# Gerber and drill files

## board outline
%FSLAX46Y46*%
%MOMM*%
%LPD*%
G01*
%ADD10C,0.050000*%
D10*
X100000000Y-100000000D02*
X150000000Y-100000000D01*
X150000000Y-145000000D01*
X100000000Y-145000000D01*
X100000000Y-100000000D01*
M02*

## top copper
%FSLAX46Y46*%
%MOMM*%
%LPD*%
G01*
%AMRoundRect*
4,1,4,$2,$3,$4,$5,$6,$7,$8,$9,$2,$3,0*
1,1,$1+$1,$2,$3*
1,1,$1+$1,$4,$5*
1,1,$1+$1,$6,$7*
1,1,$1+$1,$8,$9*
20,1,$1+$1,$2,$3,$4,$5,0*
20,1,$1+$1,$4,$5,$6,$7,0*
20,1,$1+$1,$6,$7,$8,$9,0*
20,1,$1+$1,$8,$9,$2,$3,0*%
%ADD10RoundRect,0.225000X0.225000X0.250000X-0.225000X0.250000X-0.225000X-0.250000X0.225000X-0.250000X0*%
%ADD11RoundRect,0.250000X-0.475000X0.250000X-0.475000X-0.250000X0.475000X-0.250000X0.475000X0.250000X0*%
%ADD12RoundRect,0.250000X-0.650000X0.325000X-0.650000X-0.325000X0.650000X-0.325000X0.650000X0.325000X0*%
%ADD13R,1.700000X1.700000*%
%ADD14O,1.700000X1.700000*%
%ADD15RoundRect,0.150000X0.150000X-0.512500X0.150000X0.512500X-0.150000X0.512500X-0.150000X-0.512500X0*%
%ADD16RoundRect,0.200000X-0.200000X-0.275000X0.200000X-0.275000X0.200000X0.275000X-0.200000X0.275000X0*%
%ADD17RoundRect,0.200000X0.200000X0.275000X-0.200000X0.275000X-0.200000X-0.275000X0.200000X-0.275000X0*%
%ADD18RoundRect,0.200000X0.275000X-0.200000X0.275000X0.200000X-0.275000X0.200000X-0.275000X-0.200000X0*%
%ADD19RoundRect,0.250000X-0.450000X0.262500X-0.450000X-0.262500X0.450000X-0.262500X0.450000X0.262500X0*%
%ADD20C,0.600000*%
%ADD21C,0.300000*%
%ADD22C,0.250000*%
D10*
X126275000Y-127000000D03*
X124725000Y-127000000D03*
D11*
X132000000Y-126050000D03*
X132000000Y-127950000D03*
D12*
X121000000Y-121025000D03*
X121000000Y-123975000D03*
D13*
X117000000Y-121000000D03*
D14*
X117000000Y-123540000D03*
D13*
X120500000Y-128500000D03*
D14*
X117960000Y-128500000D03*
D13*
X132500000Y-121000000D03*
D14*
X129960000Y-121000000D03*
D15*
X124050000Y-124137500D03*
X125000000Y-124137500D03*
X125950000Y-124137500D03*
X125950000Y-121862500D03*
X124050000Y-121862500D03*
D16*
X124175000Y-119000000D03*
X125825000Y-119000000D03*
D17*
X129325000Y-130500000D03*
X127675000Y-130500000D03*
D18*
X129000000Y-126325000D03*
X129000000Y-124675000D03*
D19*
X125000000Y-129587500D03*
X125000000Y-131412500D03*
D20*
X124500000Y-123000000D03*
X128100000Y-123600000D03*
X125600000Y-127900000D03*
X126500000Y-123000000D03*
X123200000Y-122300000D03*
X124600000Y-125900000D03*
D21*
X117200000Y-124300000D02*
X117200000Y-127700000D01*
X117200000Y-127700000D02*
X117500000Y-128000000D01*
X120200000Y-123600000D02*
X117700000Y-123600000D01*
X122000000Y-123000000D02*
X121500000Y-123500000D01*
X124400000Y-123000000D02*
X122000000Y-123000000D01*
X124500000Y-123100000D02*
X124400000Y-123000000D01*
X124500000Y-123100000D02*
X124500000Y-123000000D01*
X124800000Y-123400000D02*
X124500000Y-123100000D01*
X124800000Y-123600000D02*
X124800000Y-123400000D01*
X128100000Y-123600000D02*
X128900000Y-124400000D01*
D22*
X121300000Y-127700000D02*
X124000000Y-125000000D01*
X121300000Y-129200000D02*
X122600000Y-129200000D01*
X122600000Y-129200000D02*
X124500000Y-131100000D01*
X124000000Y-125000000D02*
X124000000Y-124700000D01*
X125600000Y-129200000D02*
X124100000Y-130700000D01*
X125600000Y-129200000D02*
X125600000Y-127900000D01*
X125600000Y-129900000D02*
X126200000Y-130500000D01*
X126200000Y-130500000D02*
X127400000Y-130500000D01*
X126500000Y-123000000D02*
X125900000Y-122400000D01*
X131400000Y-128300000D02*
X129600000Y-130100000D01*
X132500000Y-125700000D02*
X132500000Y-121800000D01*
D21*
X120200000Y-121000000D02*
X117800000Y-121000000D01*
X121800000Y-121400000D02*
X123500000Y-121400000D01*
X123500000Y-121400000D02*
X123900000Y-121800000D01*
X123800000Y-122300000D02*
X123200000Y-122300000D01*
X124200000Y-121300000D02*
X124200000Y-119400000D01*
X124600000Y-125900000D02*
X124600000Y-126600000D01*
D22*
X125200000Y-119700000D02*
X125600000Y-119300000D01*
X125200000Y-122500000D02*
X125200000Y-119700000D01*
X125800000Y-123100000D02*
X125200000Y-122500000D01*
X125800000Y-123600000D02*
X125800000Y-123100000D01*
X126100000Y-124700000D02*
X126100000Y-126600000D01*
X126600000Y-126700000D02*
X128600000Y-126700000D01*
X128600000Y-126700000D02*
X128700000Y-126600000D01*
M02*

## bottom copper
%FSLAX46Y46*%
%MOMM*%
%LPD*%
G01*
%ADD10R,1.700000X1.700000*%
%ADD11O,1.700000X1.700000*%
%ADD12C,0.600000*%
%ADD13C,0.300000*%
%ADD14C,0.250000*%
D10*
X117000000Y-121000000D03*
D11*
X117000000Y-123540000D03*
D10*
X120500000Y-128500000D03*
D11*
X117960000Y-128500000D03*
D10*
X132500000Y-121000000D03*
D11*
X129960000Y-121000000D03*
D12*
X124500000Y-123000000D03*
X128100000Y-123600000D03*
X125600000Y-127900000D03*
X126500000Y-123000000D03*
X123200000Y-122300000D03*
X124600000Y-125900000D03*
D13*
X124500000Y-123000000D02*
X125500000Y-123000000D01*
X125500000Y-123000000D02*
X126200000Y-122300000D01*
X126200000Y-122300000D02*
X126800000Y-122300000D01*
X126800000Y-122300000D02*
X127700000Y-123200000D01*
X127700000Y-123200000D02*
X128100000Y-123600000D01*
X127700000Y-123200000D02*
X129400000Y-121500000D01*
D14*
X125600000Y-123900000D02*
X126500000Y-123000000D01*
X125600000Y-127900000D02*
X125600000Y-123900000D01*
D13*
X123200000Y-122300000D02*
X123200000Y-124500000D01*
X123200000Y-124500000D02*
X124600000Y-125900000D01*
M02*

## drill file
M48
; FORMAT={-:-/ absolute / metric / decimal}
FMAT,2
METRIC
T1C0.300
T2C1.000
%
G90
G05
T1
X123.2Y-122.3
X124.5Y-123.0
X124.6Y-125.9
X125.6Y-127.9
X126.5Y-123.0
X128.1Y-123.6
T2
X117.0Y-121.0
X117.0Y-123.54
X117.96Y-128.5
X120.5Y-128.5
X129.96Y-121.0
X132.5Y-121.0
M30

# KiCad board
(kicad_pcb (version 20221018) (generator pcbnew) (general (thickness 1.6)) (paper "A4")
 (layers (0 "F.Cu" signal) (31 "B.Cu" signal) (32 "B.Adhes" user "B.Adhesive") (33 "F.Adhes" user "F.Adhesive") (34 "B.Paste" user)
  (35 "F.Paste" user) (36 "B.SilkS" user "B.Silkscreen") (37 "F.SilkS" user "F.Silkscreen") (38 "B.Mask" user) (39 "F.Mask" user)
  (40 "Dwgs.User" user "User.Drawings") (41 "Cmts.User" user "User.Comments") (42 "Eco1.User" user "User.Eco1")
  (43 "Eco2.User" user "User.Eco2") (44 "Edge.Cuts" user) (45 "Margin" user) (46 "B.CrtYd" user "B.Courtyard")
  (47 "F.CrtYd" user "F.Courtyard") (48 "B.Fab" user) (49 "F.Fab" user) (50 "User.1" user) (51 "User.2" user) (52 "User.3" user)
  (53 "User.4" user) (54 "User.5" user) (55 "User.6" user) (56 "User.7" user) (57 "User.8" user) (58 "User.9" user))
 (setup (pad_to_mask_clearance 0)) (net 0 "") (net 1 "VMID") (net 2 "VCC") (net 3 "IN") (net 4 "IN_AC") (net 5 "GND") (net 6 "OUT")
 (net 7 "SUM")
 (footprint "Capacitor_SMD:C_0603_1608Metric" (layer "F.Cu") (at 125.5 127 180)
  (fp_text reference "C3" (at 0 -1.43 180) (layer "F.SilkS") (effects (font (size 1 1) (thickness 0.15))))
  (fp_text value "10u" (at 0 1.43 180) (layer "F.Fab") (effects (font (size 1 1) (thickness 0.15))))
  (pad "1" smd roundrect (at -0.775 0 180) (size 0.9 0.95) (layers "F.Cu" "F.Paste" "F.Mask") (roundrect_rratio 0.25) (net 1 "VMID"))
  (pad "2" smd roundrect (at 0.775 0 180) (size 0.9 0.95) (layers "F.Cu" "F.Paste" "F.Mask") (roundrect_rratio 0.25) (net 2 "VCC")))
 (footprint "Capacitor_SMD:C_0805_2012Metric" (layer "F.Cu") (at 132 127 -90)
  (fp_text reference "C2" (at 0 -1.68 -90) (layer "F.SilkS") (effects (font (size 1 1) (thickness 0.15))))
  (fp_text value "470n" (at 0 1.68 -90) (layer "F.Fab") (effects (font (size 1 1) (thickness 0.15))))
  (pad "1" smd roundrect (at -0.95 0 270) (size 1 1.45) (layers "F.Cu" "F.Paste" "F.Mask") (roundrect_rratio 0.25) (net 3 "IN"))
  (pad "2" smd roundrect (at 0.95 0 270) (size 1 1.45) (layers "F.Cu" "F.Paste" "F.Mask") (roundrect_rratio 0.25) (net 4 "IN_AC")))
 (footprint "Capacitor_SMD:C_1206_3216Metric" (layer "F.Cu") (at 121 122.5 -90)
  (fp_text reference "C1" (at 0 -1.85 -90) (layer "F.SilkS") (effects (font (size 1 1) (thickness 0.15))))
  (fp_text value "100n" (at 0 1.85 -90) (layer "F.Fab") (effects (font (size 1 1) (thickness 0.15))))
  (pad "1" smd roundrect (at -1.475 0 270) (size 1.15 1.8) (layers "F.Cu" "F.Paste" "F.Mask") (roundrect_rratio 0.217391) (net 2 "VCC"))
  (pad "2" smd roundrect (at 1.475 0 270) (size 1.15 1.8) (layers "F.Cu" "F.Paste" "F.Mask") (roundrect_rratio 0.217391) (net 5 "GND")))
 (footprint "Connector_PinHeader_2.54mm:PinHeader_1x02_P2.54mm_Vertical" (layer "F.Cu") (at 117 121)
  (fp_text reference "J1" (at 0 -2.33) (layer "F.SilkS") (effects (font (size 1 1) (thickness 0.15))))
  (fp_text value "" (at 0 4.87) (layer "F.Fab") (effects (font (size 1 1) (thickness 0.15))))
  (pad "1" thru_hole rect (at 0 0) (size 1.7 1.7) (drill 1) (layers "*.Cu" "*.Mask") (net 2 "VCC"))
  (pad "2" thru_hole oval (at 0 2.54) (size 1.7 1.7) (drill 1) (layers "*.Cu" "*.Mask") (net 5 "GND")))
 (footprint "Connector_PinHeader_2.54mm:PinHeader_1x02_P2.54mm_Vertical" (layer "F.Cu") (at 120.5 128.5 -90)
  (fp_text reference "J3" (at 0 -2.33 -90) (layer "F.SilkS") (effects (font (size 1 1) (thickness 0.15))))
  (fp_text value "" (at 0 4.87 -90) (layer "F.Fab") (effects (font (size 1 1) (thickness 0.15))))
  (pad "1" thru_hole rect (at 0 0 270) (size 1.7 1.7) (drill 1) (layers "*.Cu" "*.Mask") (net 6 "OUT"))
  (pad "2" thru_hole oval (at 0 2.54 270) (size 1.7 1.7) (drill 1) (layers "*.Cu" "*.Mask") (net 5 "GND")))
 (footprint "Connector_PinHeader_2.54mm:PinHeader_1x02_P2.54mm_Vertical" (layer "F.Cu") (at 132.5 121 -90)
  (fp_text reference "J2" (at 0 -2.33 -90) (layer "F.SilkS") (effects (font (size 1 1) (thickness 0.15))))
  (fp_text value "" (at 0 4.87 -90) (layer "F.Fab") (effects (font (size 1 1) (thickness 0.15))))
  (pad "1" thru_hole rect (at 0 0 270) (size 1.7 1.7) (drill 1) (layers "*.Cu" "*.Mask") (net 3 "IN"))
  (pad "2" thru_hole oval (at 0 2.54 270) (size 1.7 1.7) (drill 1) (layers "*.Cu" "*.Mask") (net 5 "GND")))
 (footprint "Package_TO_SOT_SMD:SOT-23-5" (layer "F.Cu") (at 125 123 90)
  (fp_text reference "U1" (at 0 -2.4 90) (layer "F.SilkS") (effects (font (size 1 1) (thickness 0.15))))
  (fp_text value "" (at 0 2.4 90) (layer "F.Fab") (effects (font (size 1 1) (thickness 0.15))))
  (pad "1" smd roundrect (at -1.1375 -0.95 90) (size 1.325 0.6) (layers "F.Cu" "F.Paste" "F.Mask") (roundrect_rratio 0.25) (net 6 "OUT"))
  (pad "2" smd roundrect (at -1.1375 0 90) (size 1.325 0.6) (layers "F.Cu" "F.Paste" "F.Mask") (roundrect_rratio 0.25) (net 5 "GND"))
  (pad "3" smd roundrect (at -1.1375 0.95 90) (size 1.325 0.6) (layers "F.Cu" "F.Paste" "F.Mask") (roundrect_rratio 0.25) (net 1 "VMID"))
  (pad "4" smd roundrect (at 1.1375 0.95 90) (size 1.325 0.6) (layers "F.Cu" "F.Paste" "F.Mask") (roundrect_rratio 0.25) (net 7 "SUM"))
  (pad "5" smd roundrect (at 1.1375 -0.95 90) (size 1.325 0.6) (layers "F.Cu" "F.Paste" "F.Mask") (roundrect_rratio 0.25) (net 2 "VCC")))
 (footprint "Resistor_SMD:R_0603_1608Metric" (layer "F.Cu") (at 125 119)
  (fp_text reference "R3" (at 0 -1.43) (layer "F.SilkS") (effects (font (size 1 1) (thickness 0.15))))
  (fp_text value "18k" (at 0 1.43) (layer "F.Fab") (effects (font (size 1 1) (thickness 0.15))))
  (pad "1" smd roundrect (at -0.825 0) (size 0.8 0.95) (layers "F.Cu" "F.Paste" "F.Mask") (roundrect_rratio 0.25) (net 2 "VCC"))
  (pad "2" smd roundrect (at 0.825 0) (size 0.8 0.95) (layers "F.Cu" "F.Paste" "F.Mask") (roundrect_rratio 0.25) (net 1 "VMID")))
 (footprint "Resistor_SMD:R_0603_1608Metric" (layer "F.Cu") (at 128.5 130.5 180)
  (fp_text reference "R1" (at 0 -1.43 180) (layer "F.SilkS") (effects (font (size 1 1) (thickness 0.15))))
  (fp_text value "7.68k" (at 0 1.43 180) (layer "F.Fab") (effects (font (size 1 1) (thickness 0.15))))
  (pad "1" smd roundrect (at -0.825 0 180) (size 0.8 0.95) (layers "F.Cu" "F.Paste" "F.Mask") (roundrect_rratio 0.25) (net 4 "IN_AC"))
  (pad "2" smd roundrect (at 0.825 0 180) (size 0.8 0.95) (layers "F.Cu" "F.Paste" "F.Mask") (roundrect_rratio 0.25) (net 7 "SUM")))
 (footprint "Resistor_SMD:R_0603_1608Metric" (layer "F.Cu") (at 129 125.5 90)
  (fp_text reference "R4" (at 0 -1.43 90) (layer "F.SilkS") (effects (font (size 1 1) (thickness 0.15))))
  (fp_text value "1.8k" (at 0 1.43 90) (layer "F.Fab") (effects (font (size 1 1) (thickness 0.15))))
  (pad "1" smd roundrect (at -0.825 0 90) (size 0.8 0.95) (layers "F.Cu" "F.Paste" "F.Mask") (roundrect_rratio 0.25) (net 1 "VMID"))
  (pad "2" smd roundrect (at 0.825 0 90) (size 0.8 0.95) (layers "F.Cu" "F.Paste" "F.Mask") (roundrect_rratio 0.25) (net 5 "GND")))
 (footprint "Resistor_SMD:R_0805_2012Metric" (layer "F.Cu") (at 125 130.5 -90)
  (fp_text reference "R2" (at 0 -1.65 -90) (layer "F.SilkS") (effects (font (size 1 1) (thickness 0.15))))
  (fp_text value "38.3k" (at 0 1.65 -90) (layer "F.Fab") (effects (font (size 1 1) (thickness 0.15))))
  (pad "1" smd roundrect (at -0.9125 0 270) (size 1.025 1.4) (layers "F.Cu" "F.Paste" "F.Mask") (roundrect_rratio 0.243902) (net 7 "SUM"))
  (pad "2" smd roundrect (at 0.9125 0 270) (size 1.025 1.4) (layers "F.Cu" "F.Paste" "F.Mask") (roundrect_rratio 0.243902) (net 6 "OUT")))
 (gr_rect (start 100 100) (end 150 145) (stroke (width 0.05) (type default)) (fill none) (layer "Edge.Cuts"))
 (segment (start 117.2 124.3) (end 117.2 127.7) (width 0.3) (layer "F.Cu") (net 5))
 (segment (start 117.2 127.7) (end 117.5 128) (width 0.3) (layer "F.Cu") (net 5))
 (segment (start 120.2 123.6) (end 117.7 123.6) (width 0.3) (layer "F.Cu") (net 5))
 (segment (start 122 123) (end 121.5 123.5) (width 0.3) (layer "F.Cu") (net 5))
 (segment (start 124.4 123) (end 122 123) (width 0.3) (layer "F.Cu") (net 5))
 (segment (start 124.5 123.1) (end 124.4 123) (width 0.3) (layer "F.Cu") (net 5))
 (segment (start 124.5 123.1) (end 124.5 123) (width 0.3) (layer "F.Cu") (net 5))
 (segment (start 124.8 123.4) (end 124.5 123.1) (width 0.3) (layer "F.Cu") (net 5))
 (segment (start 124.8 123.6) (end 124.8 123.4) (width 0.3) (layer "F.Cu") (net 5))
 (segment (start 128.1 123.6) (end 128.9 124.4) (width 0.3) (layer "F.Cu") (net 5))
 (via (at 124.5 123) (size 0.6) (drill 0.3) (layers "F.Cu" "B.Cu") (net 5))
 (via (at 128.1 123.6) (size 0.6) (drill 0.3) (layers "F.Cu" "B.Cu") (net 5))
 (segment (start 121.3 127.7) (end 124 125) (width 0.25) (layer "F.Cu") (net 6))
 (segment (start 121.3 129.2) (end 122.6 129.2) (width 0.25) (layer "F.Cu") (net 6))
 (segment (start 122.6 129.2) (end 124.5 131.1) (width 0.25) (layer "F.Cu") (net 6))
 (segment (start 124 125) (end 124 124.7) (width 0.25) (layer "F.Cu") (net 6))
 (segment (start 124.5 123) (end 125.5 123) (width 0.3) (layer "B.Cu") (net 5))
 (segment (start 125.5 123) (end 126.2 122.3) (width 0.3) (layer "B.Cu") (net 5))
 (segment (start 125.6 129.2) (end 124.1 130.7) (width 0.25) (layer "F.Cu") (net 7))
 (segment (start 125.6 129.2) (end 125.6 127.9) (width 0.25) (layer "F.Cu") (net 7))
 (segment (start 125.6 129.9) (end 126.2 130.5) (width 0.25) (layer "F.Cu") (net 7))
 (segment (start 126.2 122.3) (end 126.8 122.3) (width 0.3) (layer "B.Cu") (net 5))
 (segment (start 126.2 130.5) (end 127.4 130.5) (width 0.25) (layer "F.Cu") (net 7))
 (segment (start 126.5 123) (end 125.9 122.4) (width 0.25) (layer "F.Cu") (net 7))
 (segment (start 126.8 122.3) (end 127.7 123.2) (width 0.3) (layer "B.Cu") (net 5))
 (segment (start 127.7 123.2) (end 128.1 123.6) (width 0.3) (layer "B.Cu") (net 5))
 (segment (start 127.7 123.2) (end 129.4 121.5) (width 0.3) (layer "B.Cu") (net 5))
 (segment (start 131.4 128.3) (end 129.6 130.1) (width 0.25) (layer "F.Cu") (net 4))
 (segment (start 132.5 125.7) (end 132.5 121.8) (width 0.25) (layer "F.Cu") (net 3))
 (via (at 125.6 127.9) (size 0.6) (drill 0.3) (layers "F.Cu" "B.Cu") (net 7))
 (via (at 126.5 123) (size 0.6) (drill 0.3) (layers "F.Cu" "B.Cu") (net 7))
 (segment (start 120.2 121) (end 117.8 121) (width 0.3) (layer "F.Cu") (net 2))
 (segment (start 121.8 121.4) (end 123.5 121.4) (width 0.3) (layer "F.Cu") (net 2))
 (segment (start 123.5 121.4) (end 123.9 121.8) (width 0.3) (layer "F.Cu") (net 2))
 (segment (start 123.8 122.3) (end 123.2 122.3) (width 0.3) (layer "F.Cu") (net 2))
 (segment (start 124.2 121.3) (end 124.2 119.4) (width 0.3) (layer "F.Cu") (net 2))
 (segment (start 124.6 125.9) (end 124.6 126.6) (width 0.3) (layer "F.Cu") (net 2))
 (segment (start 125.6 123.9) (end 126.5 123) (width 0.25) (layer "B.Cu") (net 7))
 (segment (start 125.6 127.9) (end 125.6 123.9) (width 0.25) (layer "B.Cu") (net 7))
 (via (at 123.2 122.3) (size 0.6) (drill 0.3) (layers "F.Cu" "B.Cu") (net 2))
 (via (at 124.6 125.9) (size 0.6) (drill 0.3) (layers "F.Cu" "B.Cu") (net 2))
 (segment (start 123.2 122.3) (end 123.2 124.5) (width 0.3) (layer "B.Cu") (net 2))
 (segment (start 123.2 124.5) (end 124.6 125.9) (width 0.3) (layer "B.Cu") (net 2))
 (segment (start 125.2 119.7) (end 125.6 119.3) (width 0.25) (layer "F.Cu") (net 1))
 (segment (start 125.2 122.5) (end 125.2 119.7) (width 0.25) (layer "F.Cu") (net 1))
 (segment (start 125.8 123.1) (end 125.2 122.5) (width 0.25) (layer "F.Cu") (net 1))
 (segment (start 125.8 123.6) (end 125.8 123.1) (width 0.25) (layer "F.Cu") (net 1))
 (segment (start 126.1 124.7) (end 126.1 126.6) (width 0.25) (layer "F.Cu") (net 1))
 (segment (start 126.6 126.7) (end 128.6 126.7) (width 0.25) (layer "F.Cu") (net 1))
 (segment (start 128.6 126.7) (end 128.7 126.6) (width 0.25) (layer "F.Cu") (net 1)))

